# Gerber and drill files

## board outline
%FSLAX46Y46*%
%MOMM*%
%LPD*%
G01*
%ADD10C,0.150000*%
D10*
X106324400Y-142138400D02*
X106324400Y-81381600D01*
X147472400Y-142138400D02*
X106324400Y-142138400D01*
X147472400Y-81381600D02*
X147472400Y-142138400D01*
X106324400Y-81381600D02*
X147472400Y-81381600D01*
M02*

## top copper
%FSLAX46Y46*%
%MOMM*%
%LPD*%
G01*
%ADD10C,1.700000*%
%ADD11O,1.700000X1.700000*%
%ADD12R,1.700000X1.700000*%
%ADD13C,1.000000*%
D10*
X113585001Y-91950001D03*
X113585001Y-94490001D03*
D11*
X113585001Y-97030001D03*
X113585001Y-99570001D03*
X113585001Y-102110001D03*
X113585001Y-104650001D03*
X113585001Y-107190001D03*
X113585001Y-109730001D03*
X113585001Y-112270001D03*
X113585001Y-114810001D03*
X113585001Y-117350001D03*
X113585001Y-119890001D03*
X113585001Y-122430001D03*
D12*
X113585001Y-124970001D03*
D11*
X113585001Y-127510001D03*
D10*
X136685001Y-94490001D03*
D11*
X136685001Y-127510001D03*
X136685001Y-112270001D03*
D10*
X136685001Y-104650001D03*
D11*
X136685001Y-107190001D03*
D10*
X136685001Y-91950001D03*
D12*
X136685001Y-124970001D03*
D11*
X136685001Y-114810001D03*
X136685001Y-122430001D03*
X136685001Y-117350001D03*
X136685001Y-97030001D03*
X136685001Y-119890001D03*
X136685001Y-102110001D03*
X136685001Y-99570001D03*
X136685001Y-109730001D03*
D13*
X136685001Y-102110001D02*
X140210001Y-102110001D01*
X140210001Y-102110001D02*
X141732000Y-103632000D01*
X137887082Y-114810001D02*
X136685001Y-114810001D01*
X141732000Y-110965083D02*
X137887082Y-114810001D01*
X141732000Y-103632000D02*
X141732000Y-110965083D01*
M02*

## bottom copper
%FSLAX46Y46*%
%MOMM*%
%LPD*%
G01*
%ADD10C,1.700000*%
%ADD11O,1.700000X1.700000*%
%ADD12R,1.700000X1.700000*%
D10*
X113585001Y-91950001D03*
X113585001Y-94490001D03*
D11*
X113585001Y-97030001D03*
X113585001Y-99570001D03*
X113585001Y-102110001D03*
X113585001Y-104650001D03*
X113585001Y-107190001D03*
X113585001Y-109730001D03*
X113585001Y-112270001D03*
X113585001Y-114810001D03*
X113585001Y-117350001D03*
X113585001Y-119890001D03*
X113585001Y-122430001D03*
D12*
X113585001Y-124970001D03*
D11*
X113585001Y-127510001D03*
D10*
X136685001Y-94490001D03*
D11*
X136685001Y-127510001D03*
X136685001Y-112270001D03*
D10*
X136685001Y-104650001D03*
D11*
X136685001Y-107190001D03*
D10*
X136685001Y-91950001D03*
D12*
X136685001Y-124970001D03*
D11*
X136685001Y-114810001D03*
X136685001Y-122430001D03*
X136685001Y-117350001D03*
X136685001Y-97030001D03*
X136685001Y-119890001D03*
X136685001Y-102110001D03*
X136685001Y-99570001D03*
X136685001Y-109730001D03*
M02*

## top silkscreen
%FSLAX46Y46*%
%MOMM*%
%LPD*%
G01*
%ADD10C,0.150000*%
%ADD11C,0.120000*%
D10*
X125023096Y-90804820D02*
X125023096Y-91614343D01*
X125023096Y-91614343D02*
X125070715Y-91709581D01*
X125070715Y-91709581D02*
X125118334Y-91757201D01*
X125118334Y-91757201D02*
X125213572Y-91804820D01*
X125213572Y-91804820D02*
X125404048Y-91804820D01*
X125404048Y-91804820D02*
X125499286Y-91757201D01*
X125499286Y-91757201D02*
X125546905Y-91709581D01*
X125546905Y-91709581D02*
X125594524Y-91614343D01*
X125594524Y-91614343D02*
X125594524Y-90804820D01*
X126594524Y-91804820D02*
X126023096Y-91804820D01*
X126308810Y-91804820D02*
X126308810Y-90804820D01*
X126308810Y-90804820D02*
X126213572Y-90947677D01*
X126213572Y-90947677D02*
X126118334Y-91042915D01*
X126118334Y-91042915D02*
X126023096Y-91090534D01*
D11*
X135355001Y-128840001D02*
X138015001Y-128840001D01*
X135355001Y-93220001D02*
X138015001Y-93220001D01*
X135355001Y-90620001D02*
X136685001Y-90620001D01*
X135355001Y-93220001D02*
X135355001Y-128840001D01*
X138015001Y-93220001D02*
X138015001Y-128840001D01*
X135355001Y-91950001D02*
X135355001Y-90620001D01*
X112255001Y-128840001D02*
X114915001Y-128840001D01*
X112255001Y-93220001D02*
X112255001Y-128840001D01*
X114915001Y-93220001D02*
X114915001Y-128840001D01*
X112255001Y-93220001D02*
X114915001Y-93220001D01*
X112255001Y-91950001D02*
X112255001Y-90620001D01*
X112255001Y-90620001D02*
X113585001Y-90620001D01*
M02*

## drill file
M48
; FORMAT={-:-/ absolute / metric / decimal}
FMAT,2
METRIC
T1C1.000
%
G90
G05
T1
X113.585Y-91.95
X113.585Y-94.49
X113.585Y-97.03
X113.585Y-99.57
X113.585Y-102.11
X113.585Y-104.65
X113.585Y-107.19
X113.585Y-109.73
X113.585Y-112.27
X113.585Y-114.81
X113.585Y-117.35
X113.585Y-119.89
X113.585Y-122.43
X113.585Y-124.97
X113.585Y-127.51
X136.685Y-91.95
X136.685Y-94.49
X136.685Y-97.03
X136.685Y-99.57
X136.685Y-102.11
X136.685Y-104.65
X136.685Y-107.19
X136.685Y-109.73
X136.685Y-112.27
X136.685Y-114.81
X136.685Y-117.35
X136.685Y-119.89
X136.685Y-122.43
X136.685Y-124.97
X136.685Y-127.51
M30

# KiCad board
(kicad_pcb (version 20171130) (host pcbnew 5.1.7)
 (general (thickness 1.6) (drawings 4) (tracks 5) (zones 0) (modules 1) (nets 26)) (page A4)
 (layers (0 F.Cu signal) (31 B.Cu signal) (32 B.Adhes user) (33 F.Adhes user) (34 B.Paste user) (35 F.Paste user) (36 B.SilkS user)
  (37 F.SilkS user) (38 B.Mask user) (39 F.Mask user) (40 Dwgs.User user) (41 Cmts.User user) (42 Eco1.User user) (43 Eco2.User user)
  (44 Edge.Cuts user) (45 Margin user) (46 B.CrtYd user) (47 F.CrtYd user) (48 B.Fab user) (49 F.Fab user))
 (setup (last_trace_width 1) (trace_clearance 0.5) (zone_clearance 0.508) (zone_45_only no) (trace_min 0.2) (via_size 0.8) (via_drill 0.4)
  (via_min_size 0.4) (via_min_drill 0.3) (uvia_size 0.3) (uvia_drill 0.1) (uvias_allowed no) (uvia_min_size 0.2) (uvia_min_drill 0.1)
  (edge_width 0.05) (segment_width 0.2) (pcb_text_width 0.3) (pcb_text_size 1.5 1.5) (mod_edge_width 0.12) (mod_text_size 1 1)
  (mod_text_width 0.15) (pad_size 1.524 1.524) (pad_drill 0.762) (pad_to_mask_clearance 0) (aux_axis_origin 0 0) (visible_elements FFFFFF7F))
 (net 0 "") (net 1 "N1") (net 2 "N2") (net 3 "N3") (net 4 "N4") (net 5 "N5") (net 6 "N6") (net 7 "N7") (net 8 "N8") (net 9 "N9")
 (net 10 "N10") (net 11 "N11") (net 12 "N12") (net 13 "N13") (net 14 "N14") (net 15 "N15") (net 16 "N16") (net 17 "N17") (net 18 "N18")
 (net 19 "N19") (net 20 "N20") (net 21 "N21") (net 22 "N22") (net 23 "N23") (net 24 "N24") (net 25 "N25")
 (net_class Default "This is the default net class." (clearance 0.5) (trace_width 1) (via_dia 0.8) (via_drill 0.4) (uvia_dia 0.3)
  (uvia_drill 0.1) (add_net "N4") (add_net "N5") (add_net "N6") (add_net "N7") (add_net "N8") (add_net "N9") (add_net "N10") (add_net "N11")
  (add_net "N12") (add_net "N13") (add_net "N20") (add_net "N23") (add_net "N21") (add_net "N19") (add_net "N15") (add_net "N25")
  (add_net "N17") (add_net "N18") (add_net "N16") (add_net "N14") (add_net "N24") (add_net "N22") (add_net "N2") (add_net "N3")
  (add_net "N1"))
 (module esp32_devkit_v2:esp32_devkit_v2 (layer F.Cu) (at 113.585001 91.950001)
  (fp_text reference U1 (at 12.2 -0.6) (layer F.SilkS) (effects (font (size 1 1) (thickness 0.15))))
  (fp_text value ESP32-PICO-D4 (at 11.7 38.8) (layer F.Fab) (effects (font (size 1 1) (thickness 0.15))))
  (fp_line (start 21.77 36.89) (end 24.43 36.89) (layer F.SilkS) (width 0.12))
  (fp_line (start 21.77 1.27) (end 24.43 1.27) (layer F.SilkS) (width 0.12))
  (fp_line (start 21.77 -1.33) (end 23.1 -1.33) (layer F.SilkS) (width 0.12))
  (fp_line (start 21.77 1.27) (end 21.77 36.89) (layer F.SilkS) (width 0.12))
  (fp_line (start 24.43 1.27) (end 24.43 36.89) (layer F.SilkS) (width 0.12))
  (fp_line (start 21.77 0) (end 21.77 -1.33) (layer F.SilkS) (width 0.12))
  (fp_line (start -1.33 36.89) (end 1.33 36.89) (layer F.SilkS) (width 0.12))
  (fp_line (start -1.33 1.27) (end -1.33 36.89) (layer F.SilkS) (width 0.12))
  (fp_line (start 1.33 1.27) (end 1.33 36.89) (layer F.SilkS) (width 0.12))
  (fp_line (start -1.33 1.27) (end 1.33 1.27) (layer F.SilkS) (width 0.12))
  (fp_line (start -1.33 0) (end -1.33 -1.33) (layer F.SilkS) (width 0.12))
  (fp_line (start -1.33 -1.33) (end 0 -1.33) (layer F.SilkS) (width 0.12))
  (pad 9 thru_hole circle (at 0 0) (size 1.7 1.7) (drill 1) (layers *.Cu *.Mask) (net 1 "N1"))
  (pad 5 thru_hole circle (at 0 2.54) (size 1.7 1.7) (drill 1) (layers *.Cu *.Mask) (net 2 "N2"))
  (pad 8 thru_hole oval (at 0 5.08) (size 1.7 1.7) (drill 1) (layers *.Cu *.Mask) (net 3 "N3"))
  (pad 10 thru_hole oval (at 0 7.62) (size 1.7 1.7) (drill 1) (layers *.Cu *.Mask) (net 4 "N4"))
  (pad 11 thru_hole oval (at 0 10.16) (size 1.7 1.7) (drill 1) (layers *.Cu *.Mask) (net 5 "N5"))
  (pad 12 thru_hole oval (at 0 12.7) (size 1.7 1.7) (drill 1) (layers *.Cu *.Mask) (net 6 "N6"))
  (pad 13 thru_hole oval (at 0 15.24) (size 1.7 1.7) (drill 1) (layers *.Cu *.Mask) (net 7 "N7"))
  (pad 14 thru_hole oval (at 0 17.78) (size 1.7 1.7) (drill 1) (layers *.Cu *.Mask) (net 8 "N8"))
  (pad 15 thru_hole oval (at 0 20.32) (size 1.7 1.7) (drill 1) (layers *.Cu *.Mask) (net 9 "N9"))
  (pad 16 thru_hole oval (at 0 22.86) (size 1.7 1.7) (drill 1) (layers *.Cu *.Mask) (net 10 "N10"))
  (pad 17 thru_hole oval (at 0 25.4) (size 1.7 1.7) (drill 1) (layers *.Cu *.Mask) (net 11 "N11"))
  (pad 18 thru_hole oval (at 0 27.94) (size 1.7 1.7) (drill 1) (layers *.Cu *.Mask) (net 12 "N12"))
  (pad 20 thru_hole oval (at 0 30.48) (size 1.7 1.7) (drill 1) (layers *.Cu *.Mask) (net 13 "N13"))
  (pad GND thru_hole rect (at 0 33.02) (size 1.7 1.7) (drill 1) (layers *.Cu *.Mask))
  (pad VIN thru_hole oval (at 0 35.56) (size 1.7 1.7) (drill 1) (layers *.Cu *.Mask))
  (pad 39 thru_hole circle (at 23.1 2.54) (size 1.7 1.7) (drill 1) (layers *.Cu *.Mask) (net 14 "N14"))
  (pad 3.3V thru_hole oval (at 23.1 35.56) (size 1.7 1.7) (drill 1) (layers *.Cu *.Mask))
  (pad 27 thru_hole oval (at 23.1 20.32) (size 1.7 1.7) (drill 1) (layers *.Cu *.Mask) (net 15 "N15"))
  (pad 38 thru_hole circle (at 23.1 12.7) (size 1.7 1.7) (drill 1) (layers *.Cu *.Mask) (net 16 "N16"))
  (pad 35 thru_hole oval (at 23.1 15.24) (size 1.7 1.7) (drill 1) (layers *.Cu *.Mask) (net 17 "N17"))
  (pad 36 thru_hole circle (at 23.1 0) (size 1.7 1.7) (drill 1) (layers *.Cu *.Mask) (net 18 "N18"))
  (pad GND thru_hole rect (at 23.1 33.02) (size 1.7 1.7) (drill 1) (layers *.Cu *.Mask))
  (pad 25 thru_hole oval (at 23.1 22.86) (size 1.7 1.7) (drill 1) (layers *.Cu *.Mask) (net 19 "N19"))
  (pad 21 thru_hole oval (at 23.1 30.48) (size 1.7 1.7) (drill 1) (layers *.Cu *.Mask) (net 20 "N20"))
  (pad 24 thru_hole oval (at 23.1 25.4) (size 1.7 1.7) (drill 1) (layers *.Cu *.Mask) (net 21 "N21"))
  (pad 41 thru_hole oval (at 23.1 5.08) (size 1.7 1.7) (drill 1) (layers *.Cu *.Mask) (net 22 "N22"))
  (pad 22 thru_hole oval (at 23.1 27.94) (size 1.7 1.7) (drill 1) (layers *.Cu *.Mask) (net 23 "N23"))
  (pad 42 thru_hole oval (at 23.1 10.16) (size 1.7 1.7) (drill 1) (layers *.Cu *.Mask) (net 19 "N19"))
  (pad 40 thru_hole oval (at 23.1 7.62) (size 1.7 1.7) (drill 1) (layers *.Cu *.Mask) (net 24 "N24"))
  (pad 34 thru_hole oval (at 23.1 17.78) (size 1.7 1.7) (drill 1) (layers *.Cu *.Mask) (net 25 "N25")))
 (gr_line (start 106.3244 142.1384) (end 106.3244 81.3816) (layer Edge.Cuts) (width 0.15))
 (gr_line (start 147.4724 142.1384) (end 106.3244 142.1384) (layer Edge.Cuts) (width 0.15))
 (gr_line (start 147.4724 81.3816) (end 147.4724 142.1384) (layer Edge.Cuts) (width 0.15))
 (gr_line (start 106.3244 81.3816) (end 147.4724 81.3816) (layer Edge.Cuts) (width 0.15))
 (segment (start 136.685001 102.110001) (end 140.210001 102.110001) (width 1) (layer F.Cu) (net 19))
 (segment (start 140.210001 102.110001) (end 141.732 103.632) (width 1) (layer F.Cu) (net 19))
 (segment (start 137.887082 114.810001) (end 136.685001 114.810001) (width 1) (layer F.Cu) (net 19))
 (segment (start 141.732 110.965083) (end 137.887082 114.810001) (width 1) (layer F.Cu) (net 19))
 (segment (start 141.732 103.632) (end 141.732 110.965083) (width 1) (layer F.Cu) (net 19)))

